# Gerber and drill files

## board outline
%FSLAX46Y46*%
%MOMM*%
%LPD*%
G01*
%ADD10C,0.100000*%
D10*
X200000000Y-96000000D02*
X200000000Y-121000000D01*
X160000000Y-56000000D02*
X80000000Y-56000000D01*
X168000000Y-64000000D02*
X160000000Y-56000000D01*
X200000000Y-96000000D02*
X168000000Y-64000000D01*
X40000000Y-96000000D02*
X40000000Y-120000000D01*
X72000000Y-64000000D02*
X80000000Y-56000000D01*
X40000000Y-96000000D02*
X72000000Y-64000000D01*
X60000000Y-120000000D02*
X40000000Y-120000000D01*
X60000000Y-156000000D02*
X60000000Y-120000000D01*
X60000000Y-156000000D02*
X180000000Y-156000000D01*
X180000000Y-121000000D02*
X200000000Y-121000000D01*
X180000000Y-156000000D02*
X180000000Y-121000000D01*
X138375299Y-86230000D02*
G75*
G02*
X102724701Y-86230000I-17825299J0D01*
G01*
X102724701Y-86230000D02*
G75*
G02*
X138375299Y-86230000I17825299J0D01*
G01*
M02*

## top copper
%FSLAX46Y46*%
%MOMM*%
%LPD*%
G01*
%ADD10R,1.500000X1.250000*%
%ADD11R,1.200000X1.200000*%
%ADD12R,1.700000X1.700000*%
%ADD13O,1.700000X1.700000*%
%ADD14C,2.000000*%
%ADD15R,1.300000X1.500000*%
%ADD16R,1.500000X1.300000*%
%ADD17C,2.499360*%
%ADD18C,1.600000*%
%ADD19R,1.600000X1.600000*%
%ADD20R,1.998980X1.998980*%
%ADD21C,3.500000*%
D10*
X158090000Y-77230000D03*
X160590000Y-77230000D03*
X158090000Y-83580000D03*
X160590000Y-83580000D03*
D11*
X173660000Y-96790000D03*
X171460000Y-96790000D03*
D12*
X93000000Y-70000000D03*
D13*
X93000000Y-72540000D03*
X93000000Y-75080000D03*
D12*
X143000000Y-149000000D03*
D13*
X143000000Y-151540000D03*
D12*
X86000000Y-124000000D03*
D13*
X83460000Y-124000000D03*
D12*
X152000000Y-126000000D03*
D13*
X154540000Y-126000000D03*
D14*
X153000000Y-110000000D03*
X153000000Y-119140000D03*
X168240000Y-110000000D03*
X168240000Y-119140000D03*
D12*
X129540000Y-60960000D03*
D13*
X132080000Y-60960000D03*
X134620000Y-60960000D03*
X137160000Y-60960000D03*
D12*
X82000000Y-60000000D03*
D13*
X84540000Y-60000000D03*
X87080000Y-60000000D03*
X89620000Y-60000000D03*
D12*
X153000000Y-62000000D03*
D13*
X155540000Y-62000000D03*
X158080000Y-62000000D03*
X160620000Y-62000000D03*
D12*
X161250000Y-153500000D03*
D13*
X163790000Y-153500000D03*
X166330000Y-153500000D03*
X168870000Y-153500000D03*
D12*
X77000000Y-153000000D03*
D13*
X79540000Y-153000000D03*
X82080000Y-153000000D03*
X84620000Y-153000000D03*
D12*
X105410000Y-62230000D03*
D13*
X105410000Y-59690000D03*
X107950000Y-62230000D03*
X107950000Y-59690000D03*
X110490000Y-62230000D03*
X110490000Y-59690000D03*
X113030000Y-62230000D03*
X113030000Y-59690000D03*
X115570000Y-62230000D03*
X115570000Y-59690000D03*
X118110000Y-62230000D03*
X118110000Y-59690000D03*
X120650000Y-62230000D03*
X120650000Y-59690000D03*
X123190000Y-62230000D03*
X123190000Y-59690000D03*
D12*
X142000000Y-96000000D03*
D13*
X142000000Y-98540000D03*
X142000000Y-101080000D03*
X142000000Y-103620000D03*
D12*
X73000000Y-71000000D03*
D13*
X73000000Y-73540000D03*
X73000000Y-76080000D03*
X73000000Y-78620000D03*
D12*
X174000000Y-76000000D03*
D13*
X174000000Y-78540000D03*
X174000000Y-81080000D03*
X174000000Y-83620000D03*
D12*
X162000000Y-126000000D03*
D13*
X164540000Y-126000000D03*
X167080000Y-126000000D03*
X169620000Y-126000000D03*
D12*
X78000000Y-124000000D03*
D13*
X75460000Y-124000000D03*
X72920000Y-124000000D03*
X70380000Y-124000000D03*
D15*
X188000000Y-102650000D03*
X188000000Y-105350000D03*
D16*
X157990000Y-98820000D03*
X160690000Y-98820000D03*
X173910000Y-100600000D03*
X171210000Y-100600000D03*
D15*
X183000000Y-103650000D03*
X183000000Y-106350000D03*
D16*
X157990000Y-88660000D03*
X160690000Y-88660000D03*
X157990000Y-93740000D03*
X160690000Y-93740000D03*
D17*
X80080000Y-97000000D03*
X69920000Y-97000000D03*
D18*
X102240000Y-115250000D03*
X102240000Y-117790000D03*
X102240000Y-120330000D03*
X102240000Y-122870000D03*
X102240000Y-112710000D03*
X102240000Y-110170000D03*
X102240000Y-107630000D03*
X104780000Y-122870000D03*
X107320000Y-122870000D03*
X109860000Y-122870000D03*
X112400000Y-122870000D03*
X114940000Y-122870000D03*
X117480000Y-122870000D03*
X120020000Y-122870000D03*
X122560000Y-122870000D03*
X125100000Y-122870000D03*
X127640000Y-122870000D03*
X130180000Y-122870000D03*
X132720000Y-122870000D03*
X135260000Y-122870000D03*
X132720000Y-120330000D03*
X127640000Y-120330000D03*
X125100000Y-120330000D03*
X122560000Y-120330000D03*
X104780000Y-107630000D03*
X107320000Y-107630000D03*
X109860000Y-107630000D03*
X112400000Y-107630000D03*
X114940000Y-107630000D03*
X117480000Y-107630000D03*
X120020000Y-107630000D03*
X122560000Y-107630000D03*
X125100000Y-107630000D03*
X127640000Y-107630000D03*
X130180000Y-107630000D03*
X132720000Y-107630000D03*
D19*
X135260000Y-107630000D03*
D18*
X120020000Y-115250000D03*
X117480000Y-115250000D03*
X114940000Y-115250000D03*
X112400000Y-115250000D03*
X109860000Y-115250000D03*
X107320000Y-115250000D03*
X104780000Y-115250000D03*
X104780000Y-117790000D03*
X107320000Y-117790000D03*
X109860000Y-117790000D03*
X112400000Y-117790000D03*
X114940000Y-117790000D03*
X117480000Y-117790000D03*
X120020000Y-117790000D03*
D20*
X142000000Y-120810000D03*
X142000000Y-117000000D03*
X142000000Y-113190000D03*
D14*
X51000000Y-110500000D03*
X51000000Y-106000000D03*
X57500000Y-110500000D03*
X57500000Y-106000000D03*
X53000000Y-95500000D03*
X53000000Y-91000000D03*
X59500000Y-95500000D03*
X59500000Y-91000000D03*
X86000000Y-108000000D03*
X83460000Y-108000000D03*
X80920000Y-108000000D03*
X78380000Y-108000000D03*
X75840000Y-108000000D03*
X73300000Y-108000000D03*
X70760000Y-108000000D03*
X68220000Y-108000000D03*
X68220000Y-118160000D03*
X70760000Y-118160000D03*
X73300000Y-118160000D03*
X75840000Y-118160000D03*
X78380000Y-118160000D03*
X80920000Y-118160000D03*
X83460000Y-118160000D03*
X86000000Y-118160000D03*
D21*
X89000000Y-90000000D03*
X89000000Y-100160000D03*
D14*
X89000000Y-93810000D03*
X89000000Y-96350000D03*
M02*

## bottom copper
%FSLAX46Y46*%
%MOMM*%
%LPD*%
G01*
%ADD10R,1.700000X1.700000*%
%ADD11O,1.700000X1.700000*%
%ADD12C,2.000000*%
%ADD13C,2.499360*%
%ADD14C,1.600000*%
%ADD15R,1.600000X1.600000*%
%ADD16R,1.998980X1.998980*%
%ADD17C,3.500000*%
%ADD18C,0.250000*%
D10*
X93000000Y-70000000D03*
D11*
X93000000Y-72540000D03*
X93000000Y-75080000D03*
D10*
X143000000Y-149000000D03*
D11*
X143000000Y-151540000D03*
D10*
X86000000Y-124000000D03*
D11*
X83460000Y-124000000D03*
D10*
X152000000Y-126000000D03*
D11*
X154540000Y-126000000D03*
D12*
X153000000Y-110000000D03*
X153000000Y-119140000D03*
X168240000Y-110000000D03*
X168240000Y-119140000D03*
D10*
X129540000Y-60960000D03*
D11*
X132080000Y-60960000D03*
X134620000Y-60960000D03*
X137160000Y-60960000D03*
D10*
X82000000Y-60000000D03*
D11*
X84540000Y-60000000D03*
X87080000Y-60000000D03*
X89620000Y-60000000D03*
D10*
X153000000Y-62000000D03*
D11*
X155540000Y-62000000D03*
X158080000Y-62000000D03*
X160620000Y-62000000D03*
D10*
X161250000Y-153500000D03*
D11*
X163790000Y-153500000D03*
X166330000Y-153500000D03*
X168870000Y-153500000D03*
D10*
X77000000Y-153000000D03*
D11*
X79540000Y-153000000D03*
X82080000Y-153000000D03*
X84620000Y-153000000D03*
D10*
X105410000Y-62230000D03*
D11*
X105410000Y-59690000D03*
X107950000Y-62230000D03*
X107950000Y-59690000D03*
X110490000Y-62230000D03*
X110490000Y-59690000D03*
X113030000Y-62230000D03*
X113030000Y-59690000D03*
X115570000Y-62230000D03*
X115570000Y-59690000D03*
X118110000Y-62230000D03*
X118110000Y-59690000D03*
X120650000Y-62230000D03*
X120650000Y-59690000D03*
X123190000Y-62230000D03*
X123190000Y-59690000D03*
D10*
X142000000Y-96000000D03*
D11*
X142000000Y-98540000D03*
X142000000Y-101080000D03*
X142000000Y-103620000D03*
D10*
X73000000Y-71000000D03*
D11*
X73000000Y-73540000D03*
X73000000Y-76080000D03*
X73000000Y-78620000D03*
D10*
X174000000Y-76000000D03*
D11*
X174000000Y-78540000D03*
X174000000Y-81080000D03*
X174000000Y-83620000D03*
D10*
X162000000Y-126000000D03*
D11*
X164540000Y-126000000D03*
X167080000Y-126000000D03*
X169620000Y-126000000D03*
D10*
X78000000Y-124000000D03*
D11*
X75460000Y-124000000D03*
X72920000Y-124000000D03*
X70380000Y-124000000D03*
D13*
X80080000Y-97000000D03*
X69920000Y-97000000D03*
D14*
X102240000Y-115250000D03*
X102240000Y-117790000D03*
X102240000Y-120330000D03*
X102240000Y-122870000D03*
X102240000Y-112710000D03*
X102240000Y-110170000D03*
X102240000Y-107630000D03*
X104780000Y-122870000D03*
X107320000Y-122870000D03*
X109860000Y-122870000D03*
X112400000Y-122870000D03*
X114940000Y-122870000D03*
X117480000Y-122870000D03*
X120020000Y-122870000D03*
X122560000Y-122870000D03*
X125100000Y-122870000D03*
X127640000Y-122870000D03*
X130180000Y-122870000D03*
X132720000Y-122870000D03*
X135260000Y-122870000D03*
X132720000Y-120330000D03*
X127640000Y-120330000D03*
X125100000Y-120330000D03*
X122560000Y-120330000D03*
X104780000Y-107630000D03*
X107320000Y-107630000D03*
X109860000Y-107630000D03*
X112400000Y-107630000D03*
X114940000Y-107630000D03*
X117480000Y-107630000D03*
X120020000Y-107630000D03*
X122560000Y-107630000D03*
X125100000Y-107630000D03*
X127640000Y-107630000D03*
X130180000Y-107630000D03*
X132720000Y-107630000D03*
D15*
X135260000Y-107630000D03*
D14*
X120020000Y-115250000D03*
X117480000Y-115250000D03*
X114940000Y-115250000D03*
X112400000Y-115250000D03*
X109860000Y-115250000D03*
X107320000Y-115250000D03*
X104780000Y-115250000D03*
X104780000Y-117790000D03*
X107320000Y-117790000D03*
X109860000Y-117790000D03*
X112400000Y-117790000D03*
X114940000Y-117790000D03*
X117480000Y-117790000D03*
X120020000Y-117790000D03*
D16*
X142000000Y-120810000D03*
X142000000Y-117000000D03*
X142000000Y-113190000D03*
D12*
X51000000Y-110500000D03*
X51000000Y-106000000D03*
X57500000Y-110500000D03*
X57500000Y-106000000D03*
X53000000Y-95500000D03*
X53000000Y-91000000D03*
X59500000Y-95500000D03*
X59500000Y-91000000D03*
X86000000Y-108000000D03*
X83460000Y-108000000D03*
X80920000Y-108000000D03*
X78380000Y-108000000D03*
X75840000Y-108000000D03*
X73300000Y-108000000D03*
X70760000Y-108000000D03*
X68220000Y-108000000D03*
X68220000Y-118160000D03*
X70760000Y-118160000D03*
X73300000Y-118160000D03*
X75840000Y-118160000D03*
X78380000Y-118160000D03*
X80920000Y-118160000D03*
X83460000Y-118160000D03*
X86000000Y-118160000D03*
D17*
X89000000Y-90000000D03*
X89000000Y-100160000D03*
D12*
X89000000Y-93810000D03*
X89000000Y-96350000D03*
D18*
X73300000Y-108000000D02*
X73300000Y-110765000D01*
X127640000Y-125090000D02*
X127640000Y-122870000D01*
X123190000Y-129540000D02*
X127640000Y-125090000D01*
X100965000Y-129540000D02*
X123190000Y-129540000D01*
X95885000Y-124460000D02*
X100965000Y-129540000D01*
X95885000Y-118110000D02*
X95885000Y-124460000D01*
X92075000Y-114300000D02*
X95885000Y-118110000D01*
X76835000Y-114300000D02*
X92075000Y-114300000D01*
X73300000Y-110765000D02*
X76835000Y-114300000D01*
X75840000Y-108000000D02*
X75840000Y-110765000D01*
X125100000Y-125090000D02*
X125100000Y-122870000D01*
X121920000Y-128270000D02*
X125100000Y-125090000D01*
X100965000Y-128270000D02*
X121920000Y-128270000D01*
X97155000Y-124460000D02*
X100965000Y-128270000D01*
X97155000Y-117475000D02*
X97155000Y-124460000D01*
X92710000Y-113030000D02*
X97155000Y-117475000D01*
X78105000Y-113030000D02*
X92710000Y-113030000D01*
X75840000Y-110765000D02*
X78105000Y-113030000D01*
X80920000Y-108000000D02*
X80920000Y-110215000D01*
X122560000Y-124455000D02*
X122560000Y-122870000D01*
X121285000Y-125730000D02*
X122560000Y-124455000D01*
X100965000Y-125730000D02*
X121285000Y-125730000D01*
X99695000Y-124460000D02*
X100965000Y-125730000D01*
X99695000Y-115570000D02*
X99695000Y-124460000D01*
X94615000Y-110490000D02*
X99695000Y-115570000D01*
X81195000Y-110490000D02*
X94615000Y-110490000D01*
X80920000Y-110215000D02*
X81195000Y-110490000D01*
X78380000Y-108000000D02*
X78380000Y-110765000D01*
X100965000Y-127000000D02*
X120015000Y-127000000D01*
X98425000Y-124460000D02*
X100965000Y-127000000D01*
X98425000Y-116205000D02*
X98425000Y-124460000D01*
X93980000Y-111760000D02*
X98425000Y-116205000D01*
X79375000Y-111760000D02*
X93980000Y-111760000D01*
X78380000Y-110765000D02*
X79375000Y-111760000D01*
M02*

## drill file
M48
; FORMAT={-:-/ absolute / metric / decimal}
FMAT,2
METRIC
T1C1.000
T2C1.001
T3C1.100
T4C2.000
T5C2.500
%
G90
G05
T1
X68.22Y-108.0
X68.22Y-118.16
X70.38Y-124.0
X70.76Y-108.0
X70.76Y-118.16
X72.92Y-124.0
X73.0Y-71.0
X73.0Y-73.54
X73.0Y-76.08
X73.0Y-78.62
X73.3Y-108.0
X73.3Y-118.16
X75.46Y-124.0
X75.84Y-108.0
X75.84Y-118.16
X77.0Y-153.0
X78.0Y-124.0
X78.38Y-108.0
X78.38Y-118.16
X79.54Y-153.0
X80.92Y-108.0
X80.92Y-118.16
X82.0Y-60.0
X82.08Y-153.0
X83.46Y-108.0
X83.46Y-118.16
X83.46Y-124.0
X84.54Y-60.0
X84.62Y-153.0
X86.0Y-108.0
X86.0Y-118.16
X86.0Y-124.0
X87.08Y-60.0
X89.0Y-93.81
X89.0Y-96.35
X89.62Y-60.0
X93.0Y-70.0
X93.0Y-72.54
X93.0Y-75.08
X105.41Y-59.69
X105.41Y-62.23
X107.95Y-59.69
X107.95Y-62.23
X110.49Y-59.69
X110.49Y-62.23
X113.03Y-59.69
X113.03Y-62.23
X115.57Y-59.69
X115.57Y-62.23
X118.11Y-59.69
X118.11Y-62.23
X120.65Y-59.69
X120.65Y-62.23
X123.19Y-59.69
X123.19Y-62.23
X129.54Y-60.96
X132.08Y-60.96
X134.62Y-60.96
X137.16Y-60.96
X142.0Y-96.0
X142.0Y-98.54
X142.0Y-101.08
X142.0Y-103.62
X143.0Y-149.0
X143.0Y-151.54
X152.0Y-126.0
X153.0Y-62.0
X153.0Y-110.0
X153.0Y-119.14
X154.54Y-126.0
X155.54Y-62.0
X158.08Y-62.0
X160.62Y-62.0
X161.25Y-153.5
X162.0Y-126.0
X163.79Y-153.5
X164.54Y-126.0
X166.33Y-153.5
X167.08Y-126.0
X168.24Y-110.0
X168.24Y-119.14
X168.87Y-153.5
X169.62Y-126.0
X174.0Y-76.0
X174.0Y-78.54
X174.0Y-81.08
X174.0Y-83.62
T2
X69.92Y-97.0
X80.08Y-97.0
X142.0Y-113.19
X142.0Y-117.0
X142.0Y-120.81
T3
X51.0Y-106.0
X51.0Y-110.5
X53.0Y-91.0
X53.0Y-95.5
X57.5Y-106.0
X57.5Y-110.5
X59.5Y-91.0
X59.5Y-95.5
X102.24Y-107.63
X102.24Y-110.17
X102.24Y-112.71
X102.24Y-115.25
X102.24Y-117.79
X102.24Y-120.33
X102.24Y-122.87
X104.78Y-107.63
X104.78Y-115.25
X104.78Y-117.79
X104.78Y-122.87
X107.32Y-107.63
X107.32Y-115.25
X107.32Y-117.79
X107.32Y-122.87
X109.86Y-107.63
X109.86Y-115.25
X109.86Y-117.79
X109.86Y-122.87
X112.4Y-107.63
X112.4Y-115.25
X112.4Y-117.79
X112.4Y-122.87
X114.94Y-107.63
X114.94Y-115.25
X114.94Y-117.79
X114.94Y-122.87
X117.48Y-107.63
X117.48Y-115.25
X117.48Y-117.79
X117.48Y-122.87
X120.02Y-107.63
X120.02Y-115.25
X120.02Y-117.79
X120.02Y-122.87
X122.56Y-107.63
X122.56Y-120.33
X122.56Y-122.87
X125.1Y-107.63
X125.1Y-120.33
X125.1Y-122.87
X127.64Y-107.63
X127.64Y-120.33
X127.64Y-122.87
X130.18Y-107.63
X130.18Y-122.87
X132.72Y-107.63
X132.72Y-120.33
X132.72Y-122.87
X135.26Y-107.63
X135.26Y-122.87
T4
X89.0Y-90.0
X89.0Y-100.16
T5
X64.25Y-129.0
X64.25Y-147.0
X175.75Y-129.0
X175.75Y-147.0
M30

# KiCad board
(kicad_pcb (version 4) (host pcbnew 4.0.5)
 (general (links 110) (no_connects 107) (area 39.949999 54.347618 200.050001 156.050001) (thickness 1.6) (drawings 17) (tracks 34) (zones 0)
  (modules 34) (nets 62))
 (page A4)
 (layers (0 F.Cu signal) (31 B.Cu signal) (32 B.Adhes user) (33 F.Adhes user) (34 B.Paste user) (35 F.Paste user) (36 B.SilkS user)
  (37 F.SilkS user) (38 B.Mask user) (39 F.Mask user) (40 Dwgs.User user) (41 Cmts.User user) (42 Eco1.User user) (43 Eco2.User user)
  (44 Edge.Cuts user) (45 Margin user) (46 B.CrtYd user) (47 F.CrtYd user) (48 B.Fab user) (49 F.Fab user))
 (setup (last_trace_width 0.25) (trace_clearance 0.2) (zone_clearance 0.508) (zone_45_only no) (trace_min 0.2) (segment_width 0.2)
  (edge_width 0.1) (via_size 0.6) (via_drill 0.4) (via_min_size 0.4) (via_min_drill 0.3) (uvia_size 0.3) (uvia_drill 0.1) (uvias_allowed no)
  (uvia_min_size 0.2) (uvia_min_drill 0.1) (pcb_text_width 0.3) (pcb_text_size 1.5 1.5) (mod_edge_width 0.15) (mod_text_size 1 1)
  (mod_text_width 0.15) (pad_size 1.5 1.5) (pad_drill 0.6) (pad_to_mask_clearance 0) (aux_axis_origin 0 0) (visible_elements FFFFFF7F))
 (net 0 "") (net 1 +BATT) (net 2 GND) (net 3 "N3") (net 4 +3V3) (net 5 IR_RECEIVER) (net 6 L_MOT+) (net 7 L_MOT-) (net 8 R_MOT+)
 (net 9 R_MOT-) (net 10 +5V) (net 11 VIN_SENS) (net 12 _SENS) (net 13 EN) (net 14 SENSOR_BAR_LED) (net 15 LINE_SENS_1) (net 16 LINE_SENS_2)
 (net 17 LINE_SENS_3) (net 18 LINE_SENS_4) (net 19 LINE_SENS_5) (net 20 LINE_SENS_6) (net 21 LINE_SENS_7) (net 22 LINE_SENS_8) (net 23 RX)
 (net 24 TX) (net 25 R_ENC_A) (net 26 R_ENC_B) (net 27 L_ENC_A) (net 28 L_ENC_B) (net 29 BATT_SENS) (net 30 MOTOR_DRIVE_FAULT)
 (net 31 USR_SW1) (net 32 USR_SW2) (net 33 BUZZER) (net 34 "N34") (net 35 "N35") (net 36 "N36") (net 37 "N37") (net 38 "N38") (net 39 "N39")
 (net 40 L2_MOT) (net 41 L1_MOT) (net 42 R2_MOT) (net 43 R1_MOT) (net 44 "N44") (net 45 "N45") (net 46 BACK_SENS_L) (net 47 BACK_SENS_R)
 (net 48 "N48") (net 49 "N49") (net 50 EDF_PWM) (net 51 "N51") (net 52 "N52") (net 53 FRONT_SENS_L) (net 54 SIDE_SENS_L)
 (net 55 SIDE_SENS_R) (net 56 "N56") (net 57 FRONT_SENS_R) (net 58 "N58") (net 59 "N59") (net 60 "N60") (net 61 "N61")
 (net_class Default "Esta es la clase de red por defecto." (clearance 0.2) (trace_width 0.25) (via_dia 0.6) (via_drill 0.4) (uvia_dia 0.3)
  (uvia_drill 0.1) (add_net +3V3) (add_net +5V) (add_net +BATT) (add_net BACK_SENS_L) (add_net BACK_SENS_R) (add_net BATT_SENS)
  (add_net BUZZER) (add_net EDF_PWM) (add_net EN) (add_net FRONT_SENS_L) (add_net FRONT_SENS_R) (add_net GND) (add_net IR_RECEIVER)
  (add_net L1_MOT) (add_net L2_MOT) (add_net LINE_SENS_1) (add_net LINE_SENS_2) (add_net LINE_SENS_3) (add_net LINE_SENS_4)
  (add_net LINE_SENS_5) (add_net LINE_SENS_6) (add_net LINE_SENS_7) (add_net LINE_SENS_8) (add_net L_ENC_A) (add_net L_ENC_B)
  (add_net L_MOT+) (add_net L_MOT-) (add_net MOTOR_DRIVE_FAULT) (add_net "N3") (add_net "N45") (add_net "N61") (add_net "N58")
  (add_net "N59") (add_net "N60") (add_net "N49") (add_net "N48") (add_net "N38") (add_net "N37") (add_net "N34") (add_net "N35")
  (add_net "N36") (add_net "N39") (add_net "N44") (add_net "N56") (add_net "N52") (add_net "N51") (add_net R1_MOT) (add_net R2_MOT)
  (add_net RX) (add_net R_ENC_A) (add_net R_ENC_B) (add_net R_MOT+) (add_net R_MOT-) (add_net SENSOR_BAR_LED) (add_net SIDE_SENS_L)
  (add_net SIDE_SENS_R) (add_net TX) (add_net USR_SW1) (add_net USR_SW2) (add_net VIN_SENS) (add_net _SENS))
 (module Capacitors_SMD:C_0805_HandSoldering (layer F.Cu) (at 159.34 77.23)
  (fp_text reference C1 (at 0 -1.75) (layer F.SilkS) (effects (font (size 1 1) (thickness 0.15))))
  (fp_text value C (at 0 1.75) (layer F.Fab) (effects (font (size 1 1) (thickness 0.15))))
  (pad 1 smd rect (at -1.25 0) (size 1.5 1.25) (layers F.Cu F.Paste F.Mask) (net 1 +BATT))
  (pad 2 smd rect (at 1.25 0) (size 1.5 1.25) (layers F.Cu F.Paste F.Mask) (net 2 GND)))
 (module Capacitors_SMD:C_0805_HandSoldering (layer F.Cu) (at 159.34 83.58)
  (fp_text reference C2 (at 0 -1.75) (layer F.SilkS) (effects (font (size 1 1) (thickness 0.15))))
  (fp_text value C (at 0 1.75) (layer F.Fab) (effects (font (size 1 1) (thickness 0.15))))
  (pad 1 smd rect (at -1.25 0) (size 1.5 1.25) (layers F.Cu F.Paste F.Mask) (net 1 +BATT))
  (pad 2 smd rect (at 1.25 0) (size 1.5 1.25) (layers F.Cu F.Paste F.Mask) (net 2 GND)))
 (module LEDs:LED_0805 (layer F.Cu) (at 172.56 96.79)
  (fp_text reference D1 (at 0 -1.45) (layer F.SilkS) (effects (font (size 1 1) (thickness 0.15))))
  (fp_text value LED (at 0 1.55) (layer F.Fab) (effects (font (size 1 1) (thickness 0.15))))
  (pad 2 smd rect (at 1.1 0 180) (size 1.2 1.2) (layers F.Cu F.Paste F.Mask) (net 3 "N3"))
  (pad 1 smd rect (at -1.1 0 180) (size 1.2 1.2) (layers F.Cu F.Paste F.Mask) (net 1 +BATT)))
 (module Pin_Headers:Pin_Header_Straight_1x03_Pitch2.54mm (layer F.Cu) (at 93 70)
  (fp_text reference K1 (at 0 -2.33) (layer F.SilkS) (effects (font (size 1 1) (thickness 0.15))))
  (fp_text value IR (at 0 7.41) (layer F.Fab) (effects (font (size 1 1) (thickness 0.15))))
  (pad 1 thru_hole rect (at 0 0) (size 1.7 1.7) (drill 1) (layers *.Cu *.Mask) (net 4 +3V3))
  (pad 2 thru_hole oval (at 0 2.54) (size 1.7 1.7) (drill 1) (layers *.Cu *.Mask) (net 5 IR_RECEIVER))
  (pad 3 thru_hole oval (at 0 5.08) (size 1.7 1.7) (drill 1) (layers *.Cu *.Mask) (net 2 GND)))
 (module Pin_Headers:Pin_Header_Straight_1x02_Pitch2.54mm (layer F.Cu) (at 143 149)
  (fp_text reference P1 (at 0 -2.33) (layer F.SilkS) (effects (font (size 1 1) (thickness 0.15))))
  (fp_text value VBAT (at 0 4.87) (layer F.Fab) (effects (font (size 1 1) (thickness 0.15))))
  (pad 1 thru_hole rect (at 0 0) (size 1.7 1.7) (drill 1) (layers *.Cu *.Mask) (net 1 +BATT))
  (pad 2 thru_hole oval (at 0 2.54) (size 1.7 1.7) (drill 1) (layers *.Cu *.Mask) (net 2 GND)))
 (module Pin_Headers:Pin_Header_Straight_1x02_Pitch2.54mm (layer F.Cu) (at 86 124 270)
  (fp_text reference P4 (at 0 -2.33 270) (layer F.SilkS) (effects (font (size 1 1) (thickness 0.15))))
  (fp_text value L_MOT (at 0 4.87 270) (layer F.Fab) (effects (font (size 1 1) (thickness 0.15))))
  (pad 1 thru_hole rect (at 0 0 270) (size 1.7 1.7) (drill 1) (layers *.Cu *.Mask) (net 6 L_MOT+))
  (pad 2 thru_hole oval (at 0 2.54 270) (size 1.7 1.7) (drill 1) (layers *.Cu *.Mask) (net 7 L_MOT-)))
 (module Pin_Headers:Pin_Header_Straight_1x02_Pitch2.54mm (layer F.Cu) (at 152 126 90)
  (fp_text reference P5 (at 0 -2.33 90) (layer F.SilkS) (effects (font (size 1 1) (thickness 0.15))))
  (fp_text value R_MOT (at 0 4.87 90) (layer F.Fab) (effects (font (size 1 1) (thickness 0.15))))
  (pad 1 thru_hole rect (at 0 0 90) (size 1.7 1.7) (drill 1) (layers *.Cu *.Mask) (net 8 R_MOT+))
  (pad 2 thru_hole oval (at 0 2.54 90) (size 1.7 1.7) (drill 1) (layers *.Cu *.Mask) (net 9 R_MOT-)))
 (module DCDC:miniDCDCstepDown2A (layer F.Cu) (at 153 110)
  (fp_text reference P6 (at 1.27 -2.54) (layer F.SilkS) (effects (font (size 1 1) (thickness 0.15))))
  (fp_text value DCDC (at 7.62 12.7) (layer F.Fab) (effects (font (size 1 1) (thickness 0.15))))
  (pad 2 thru_hole circle (at 0 0) (size 2 2) (drill 1) (layers *.Cu *.Mask) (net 2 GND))
  (pad 1 thru_hole circle (at 0 9.14) (size 2 2) (drill 1) (layers *.Cu *.Mask) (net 1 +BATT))
  (pad 4 thru_hole circle (at 15.24 0) (size 2 2) (drill 1) (layers *.Cu *.Mask) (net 2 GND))
  (pad 3 thru_hole circle (at 15.24 9.14) (size 2 2) (drill 1) (layers *.Cu *.Mask) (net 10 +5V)))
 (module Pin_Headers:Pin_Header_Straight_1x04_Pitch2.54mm (layer F.Cu) (at 129.54 60.96 90)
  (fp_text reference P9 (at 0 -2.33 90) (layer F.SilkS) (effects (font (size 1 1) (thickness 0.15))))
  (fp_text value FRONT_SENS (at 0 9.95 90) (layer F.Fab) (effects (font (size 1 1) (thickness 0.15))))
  (pad 1 thru_hole rect (at 0 0 90) (size 1.7 1.7) (drill 1) (layers *.Cu *.Mask) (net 2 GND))
  (pad 2 thru_hole oval (at 0 2.54 90) (size 1.7 1.7) (drill 1) (layers *.Cu *.Mask) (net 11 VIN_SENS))
  (pad 3 thru_hole oval (at 0 5.08 90) (size 1.7 1.7) (drill 1) (layers *.Cu *.Mask) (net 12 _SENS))
  (pad 4 thru_hole oval (at 0 7.62 90) (size 1.7 1.7) (drill 1) (layers *.Cu *.Mask) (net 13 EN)))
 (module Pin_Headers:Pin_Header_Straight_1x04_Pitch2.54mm (layer F.Cu) (at 82 60 90)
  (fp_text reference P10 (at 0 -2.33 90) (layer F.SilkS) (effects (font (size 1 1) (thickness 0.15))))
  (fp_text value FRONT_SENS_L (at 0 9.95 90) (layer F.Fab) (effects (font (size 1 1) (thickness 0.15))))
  (pad 1 thru_hole rect (at 0 0 90) (size 1.7 1.7) (drill 1) (layers *.Cu *.Mask) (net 2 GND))
  (pad 2 thru_hole oval (at 0 2.54 90) (size 1.7 1.7) (drill 1) (layers *.Cu *.Mask) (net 11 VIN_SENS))
  (pad 3 thru_hole oval (at 0 5.08 90) (size 1.7 1.7) (drill 1) (layers *.Cu *.Mask) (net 12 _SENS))
  (pad 4 thru_hole oval (at 0 7.62 90) (size 1.7 1.7) (drill 1) (layers *.Cu *.Mask) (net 13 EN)))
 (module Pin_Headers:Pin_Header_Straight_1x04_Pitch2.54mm (layer F.Cu) (at 153 62 90)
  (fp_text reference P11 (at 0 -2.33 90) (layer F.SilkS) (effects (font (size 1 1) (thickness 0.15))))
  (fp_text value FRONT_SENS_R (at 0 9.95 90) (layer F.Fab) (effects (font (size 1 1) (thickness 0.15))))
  (pad 1 thru_hole rect (at 0 0 90) (size 1.7 1.7) (drill 1) (layers *.Cu *.Mask) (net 2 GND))
  (pad 2 thru_hole oval (at 0 2.54 90) (size 1.7 1.7) (drill 1) (layers *.Cu *.Mask) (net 11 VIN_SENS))
  (pad 3 thru_hole oval (at 0 5.08 90) (size 1.7 1.7) (drill 1) (layers *.Cu *.Mask) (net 12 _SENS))
  (pad 4 thru_hole oval (at 0 7.62 90) (size 1.7 1.7) (drill 1) (layers *.Cu *.Mask) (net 13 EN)))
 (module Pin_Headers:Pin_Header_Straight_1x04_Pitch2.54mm (layer F.Cu) (at 161.25 153.5 90)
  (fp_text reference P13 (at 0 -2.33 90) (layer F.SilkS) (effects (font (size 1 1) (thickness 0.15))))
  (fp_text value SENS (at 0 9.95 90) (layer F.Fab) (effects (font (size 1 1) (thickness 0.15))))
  (pad 1 thru_hole rect (at 0 0 90) (size 1.7 1.7) (drill 1) (layers *.Cu *.Mask) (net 2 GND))
  (pad 2 thru_hole oval (at 0 2.54 90) (size 1.7 1.7) (drill 1) (layers *.Cu *.Mask) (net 11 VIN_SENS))
  (pad 3 thru_hole oval (at 0 5.08 90) (size 1.7 1.7) (drill 1) (layers *.Cu *.Mask) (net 12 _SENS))
  (pad 4 thru_hole oval (at 0 7.62 90) (size 1.7 1.7) (drill 1) (layers *.Cu *.Mask) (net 13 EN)))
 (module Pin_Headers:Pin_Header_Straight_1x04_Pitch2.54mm (layer F.Cu) (at 77 153 90)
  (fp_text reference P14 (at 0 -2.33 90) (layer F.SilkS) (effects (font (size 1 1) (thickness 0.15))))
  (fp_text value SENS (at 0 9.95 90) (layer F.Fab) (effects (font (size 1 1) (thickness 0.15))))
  (pad 1 thru_hole rect (at 0 0 90) (size 1.7 1.7) (drill 1) (layers *.Cu *.Mask) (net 2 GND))
  (pad 2 thru_hole oval (at 0 2.54 90) (size 1.7 1.7) (drill 1) (layers *.Cu *.Mask) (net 11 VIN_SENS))
  (pad 3 thru_hole oval (at 0 5.08 90) (size 1.7 1.7) (drill 1) (layers *.Cu *.Mask) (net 12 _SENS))
  (pad 4 thru_hole oval (at 0 7.62 90) (size 1.7 1.7) (drill 1) (layers *.Cu *.Mask) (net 13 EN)))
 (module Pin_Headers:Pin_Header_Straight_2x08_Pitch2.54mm (layer F.Cu) (at 105.41 62.23 90)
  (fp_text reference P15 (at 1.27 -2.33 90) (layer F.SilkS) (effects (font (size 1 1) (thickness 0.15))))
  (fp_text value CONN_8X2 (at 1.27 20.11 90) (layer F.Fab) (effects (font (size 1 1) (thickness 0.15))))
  (pad 1 thru_hole rect (at 0 0 90) (size 1.7 1.7) (drill 1) (layers *.Cu *.Mask) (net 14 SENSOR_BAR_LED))
  (pad 2 thru_hole oval (at 2.54 0 90) (size 1.7 1.7) (drill 1) (layers *.Cu *.Mask) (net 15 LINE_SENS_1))
  (pad 3 thru_hole oval (at 0 2.54 90) (size 1.7 1.7) (drill 1) (layers *.Cu *.Mask) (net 4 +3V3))
  (pad 4 thru_hole oval (at 2.54 2.54 90) (size 1.7 1.7) (drill 1) (layers *.Cu *.Mask) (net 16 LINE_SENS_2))
  (pad 5 thru_hole oval (at 0 5.08 90) (size 1.7 1.7) (drill 1) (layers *.Cu *.Mask) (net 2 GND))
  (pad 6 thru_hole oval (at 2.54 5.08 90) (size 1.7 1.7) (drill 1) (layers *.Cu *.Mask) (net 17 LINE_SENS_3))
  (pad 7 thru_hole oval (at 0 7.62 90) (size 1.7 1.7) (drill 1) (layers *.Cu *.Mask) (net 2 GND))
  (pad 8 thru_hole oval (at 2.54 7.62 90) (size 1.7 1.7) (drill 1) (layers *.Cu *.Mask) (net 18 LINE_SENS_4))
  (pad 9 thru_hole oval (at 0 10.16 90) (size 1.7 1.7) (drill 1) (layers *.Cu *.Mask) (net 2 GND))
  (pad 10 thru_hole oval (at 2.54 10.16 90) (size 1.7 1.7) (drill 1) (layers *.Cu *.Mask) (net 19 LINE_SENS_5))
  (pad 11 thru_hole oval (at 0 12.7 90) (size 1.7 1.7) (drill 1) (layers *.Cu *.Mask) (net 2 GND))
  (pad 12 thru_hole oval (at 2.54 12.7 90) (size 1.7 1.7) (drill 1) (layers *.Cu *.Mask) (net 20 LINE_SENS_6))
  (pad 13 thru_hole oval (at 0 15.24 90) (size 1.7 1.7) (drill 1) (layers *.Cu *.Mask) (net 2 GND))
  (pad 14 thru_hole oval (at 2.54 15.24 90) (size 1.7 1.7) (drill 1) (layers *.Cu *.Mask) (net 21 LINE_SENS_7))
  (pad 15 thru_hole oval (at 0 17.78 90) (size 1.7 1.7) (drill 1) (layers *.Cu *.Mask) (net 2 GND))
  (pad 16 thru_hole oval (at 2.54 17.78 90) (size 1.7 1.7) (drill 1) (layers *.Cu *.Mask) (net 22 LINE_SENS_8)))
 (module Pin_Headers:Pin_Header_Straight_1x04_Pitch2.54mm (layer F.Cu) (at 142 96)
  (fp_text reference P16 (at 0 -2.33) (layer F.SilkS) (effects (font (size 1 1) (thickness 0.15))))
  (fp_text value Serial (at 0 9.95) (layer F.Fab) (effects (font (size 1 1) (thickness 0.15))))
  (pad 1 thru_hole rect (at 0 0) (size 1.7 1.7) (drill 1) (layers *.Cu *.Mask) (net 10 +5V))
  (pad 2 thru_hole oval (at 0 2.54) (size 1.7 1.7) (drill 1) (layers *.Cu *.Mask) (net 2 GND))
  (pad 3 thru_hole oval (at 0 5.08) (size 1.7 1.7) (drill 1) (layers *.Cu *.Mask) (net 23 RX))
  (pad 4 thru_hole oval (at 0 7.62) (size 1.7 1.7) (drill 1) (layers *.Cu *.Mask) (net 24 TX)))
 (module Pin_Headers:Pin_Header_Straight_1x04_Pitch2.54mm (layer F.Cu) (at 73 71)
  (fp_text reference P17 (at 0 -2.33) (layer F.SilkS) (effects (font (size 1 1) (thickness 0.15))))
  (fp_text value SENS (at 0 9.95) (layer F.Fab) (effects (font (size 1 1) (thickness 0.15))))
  (pad 1 thru_hole rect (at 0 0) (size 1.7 1.7) (drill 1) (layers *.Cu *.Mask) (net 2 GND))
  (pad 2 thru_hole oval (at 0 2.54) (size 1.7 1.7) (drill 1) (layers *.Cu *.Mask) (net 11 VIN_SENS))
  (pad 3 thru_hole oval (at 0 5.08) (size 1.7 1.7) (drill 1) (layers *.Cu *.Mask) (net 12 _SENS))
  (pad 4 thru_hole oval (at 0 7.62) (size 1.7 1.7) (drill 1) (layers *.Cu *.Mask) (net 13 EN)))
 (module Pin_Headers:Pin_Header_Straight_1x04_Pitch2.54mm (layer F.Cu) (at 174 76)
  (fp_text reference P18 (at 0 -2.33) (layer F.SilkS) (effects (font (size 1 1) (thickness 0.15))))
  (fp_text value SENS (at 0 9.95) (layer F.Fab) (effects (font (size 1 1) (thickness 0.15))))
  (pad 1 thru_hole rect (at 0 0) (size 1.7 1.7) (drill 1) (layers *.Cu *.Mask) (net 2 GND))
  (pad 2 thru_hole oval (at 0 2.54) (size 1.7 1.7) (drill 1) (layers *.Cu *.Mask) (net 11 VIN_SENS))
  (pad 3 thru_hole oval (at 0 5.08) (size 1.7 1.7) (drill 1) (layers *.Cu *.Mask) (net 12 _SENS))
  (pad 4 thru_hole oval (at 0 7.62) (size 1.7 1.7) (drill 1) (layers *.Cu *.Mask) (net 13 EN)))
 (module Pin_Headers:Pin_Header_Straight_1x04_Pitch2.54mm (layer F.Cu) (at 162 126 90)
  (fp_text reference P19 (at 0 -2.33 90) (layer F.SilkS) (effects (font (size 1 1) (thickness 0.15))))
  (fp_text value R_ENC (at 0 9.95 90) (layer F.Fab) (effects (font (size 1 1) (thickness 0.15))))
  (pad 1 thru_hole rect (at 0 0 90) (size 1.7 1.7) (drill 1) (layers *.Cu *.Mask) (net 4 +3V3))
  (pad 2 thru_hole oval (at 0 2.54 90) (size 1.7 1.7) (drill 1) (layers *.Cu *.Mask) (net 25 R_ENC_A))
  (pad 3 thru_hole oval (at 0 5.08 90) (size 1.7 1.7) (drill 1) (layers *.Cu *.Mask) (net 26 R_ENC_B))
  (pad 4 thru_hole oval (at 0 7.62 90) (size 1.7 1.7) (drill 1) (layers *.Cu *.Mask) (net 2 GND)))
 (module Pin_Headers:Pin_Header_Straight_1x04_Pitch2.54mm (layer F.Cu) (at 78 124 270)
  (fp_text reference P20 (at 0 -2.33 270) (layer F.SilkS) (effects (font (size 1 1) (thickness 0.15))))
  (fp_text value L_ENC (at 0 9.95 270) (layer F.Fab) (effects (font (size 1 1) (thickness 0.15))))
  (pad 1 thru_hole rect (at 0 0 270) (size 1.7 1.7) (drill 1) (layers *.Cu *.Mask) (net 4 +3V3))
  (pad 2 thru_hole oval (at 0 2.54 270) (size 1.7 1.7) (drill 1) (layers *.Cu *.Mask) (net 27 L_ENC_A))
  (pad 3 thru_hole oval (at 0 5.08 270) (size 1.7 1.7) (drill 1) (layers *.Cu *.Mask) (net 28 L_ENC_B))
  (pad 4 thru_hole oval (at 0 7.62 270) (size 1.7 1.7) (drill 1) (layers *.Cu *.Mask) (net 2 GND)))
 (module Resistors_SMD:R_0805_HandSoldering (layer F.Cu) (at 188 104 270)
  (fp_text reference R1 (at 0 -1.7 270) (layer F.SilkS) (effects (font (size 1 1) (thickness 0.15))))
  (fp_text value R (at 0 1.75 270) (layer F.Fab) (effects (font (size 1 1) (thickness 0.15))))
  (pad 1 smd rect (at -1.35 0 270) (size 1.5 1.3) (layers F.Cu F.Paste F.Mask) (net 1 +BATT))
  (pad 2 smd rect (at 1.35 0 270) (size 1.5 1.3) (layers F.Cu F.Paste F.Mask) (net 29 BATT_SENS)))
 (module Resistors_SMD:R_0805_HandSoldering (layer F.Cu) (at 159.34 98.82)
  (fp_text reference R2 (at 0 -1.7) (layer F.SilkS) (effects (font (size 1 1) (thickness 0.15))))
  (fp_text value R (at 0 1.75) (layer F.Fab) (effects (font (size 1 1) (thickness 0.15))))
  (pad 1 smd rect (at -1.35 0) (size 1.5 1.3) (layers F.Cu F.Paste F.Mask) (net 4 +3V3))
  (pad 2 smd rect (at 1.35 0) (size 1.5 1.3) (layers F.Cu F.Paste F.Mask) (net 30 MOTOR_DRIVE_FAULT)))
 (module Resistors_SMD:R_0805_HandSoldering (layer F.Cu) (at 172.56 100.6 180)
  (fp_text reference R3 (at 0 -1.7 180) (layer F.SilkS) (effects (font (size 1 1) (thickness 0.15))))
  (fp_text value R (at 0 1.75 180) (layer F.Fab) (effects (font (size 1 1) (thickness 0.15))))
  (pad 1 smd rect (at -1.35 0 180) (size 1.5 1.3) (layers F.Cu F.Paste F.Mask) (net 3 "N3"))
  (pad 2 smd rect (at 1.35 0 180) (size 1.5 1.3) (layers F.Cu F.Paste F.Mask) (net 2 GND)))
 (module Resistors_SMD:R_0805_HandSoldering (layer F.Cu) (at 183 105 270)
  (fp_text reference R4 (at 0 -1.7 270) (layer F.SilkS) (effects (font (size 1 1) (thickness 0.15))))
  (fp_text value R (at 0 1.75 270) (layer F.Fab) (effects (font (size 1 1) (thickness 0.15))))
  (pad 1 smd rect (at -1.35 0 270) (size 1.5 1.3) (layers F.Cu F.Paste F.Mask) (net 29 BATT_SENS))
  (pad 2 smd rect (at 1.35 0 270) (size 1.5 1.3) (layers F.Cu F.Paste F.Mask) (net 2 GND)))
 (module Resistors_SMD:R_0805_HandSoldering (layer F.Cu) (at 159.34 88.66)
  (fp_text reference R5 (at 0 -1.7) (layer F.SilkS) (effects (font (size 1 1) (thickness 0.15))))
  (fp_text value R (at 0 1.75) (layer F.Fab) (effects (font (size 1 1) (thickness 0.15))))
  (pad 1 smd rect (at -1.35 0) (size 1.5 1.3) (layers F.Cu F.Paste F.Mask) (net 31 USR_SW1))
  (pad 2 smd rect (at 1.35 0) (size 1.5 1.3) (layers F.Cu F.Paste F.Mask) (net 2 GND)))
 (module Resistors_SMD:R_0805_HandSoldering (layer F.Cu) (at 159.34 93.74)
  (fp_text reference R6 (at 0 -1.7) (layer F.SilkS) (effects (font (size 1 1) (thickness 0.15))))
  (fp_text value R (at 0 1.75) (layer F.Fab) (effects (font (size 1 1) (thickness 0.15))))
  (pad 1 smd rect (at -1.35 0) (size 1.5 1.3) (layers F.Cu F.Paste F.Mask) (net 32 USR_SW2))
  (pad 2 smd rect (at 1.35 0) (size 1.5 1.3) (layers F.Cu F.Paste F.Mask) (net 2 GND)))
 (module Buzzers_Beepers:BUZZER (layer F.Cu) (at 75 97)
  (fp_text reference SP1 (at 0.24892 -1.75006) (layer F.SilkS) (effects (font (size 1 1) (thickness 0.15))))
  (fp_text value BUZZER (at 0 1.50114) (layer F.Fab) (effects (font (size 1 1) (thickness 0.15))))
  (pad 2 thru_hole circle (at 5.08 0) (size 2.49936 2.49936) (drill 1.00076) (layers *.Cu *.Mask) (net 2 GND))
  (pad 1 thru_hole circle (at -5.08 0) (size 2.49936 2.49936) (drill 1.00076) (layers *.Cu *.Mask) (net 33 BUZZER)))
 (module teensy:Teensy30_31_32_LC (layer F.Cu) (at 118.75 115.25 180)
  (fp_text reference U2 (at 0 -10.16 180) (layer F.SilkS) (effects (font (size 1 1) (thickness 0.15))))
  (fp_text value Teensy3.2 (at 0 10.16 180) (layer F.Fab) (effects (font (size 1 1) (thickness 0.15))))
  (pad 17 thru_hole circle (at 16.51 0 180) (size 1.6 1.6) (drill 1.1) (layers *.Cu *.Mask F.SilkS) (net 2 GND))
  (pad 18 thru_hole circle (at 16.51 -2.54 180) (size 1.6 1.6) (drill 1.1) (layers *.Cu *.Mask F.SilkS) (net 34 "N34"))
  (pad 19 thru_hole circle (at 16.51 -5.08 180) (size 1.6 1.6) (drill 1.1) (layers *.Cu *.Mask F.SilkS) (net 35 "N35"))
  (pad 20 thru_hole circle (at 16.51 -7.62 180) (size 1.6 1.6) (drill 1.1) (layers *.Cu *.Mask F.SilkS) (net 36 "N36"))
  (pad 16 thru_hole circle (at 16.51 2.54 180) (size 1.6 1.6) (drill 1.1) (layers *.Cu *.Mask F.SilkS) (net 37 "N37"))
  (pad 15 thru_hole circle (at 16.51 5.08 180) (size 1.6 1.6) (drill 1.1) (layers *.Cu *.Mask F.SilkS) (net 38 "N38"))
  (pad 14 thru_hole circle (at 16.51 7.62 180) (size 1.6 1.6) (drill 1.1) (layers *.Cu *.Mask F.SilkS) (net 30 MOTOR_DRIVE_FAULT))
  (pad 21 thru_hole circle (at 13.97 -7.62 180) (size 1.6 1.6) (drill 1.1) (layers *.Cu *.Mask F.SilkS) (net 29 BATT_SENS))
  (pad 22 thru_hole circle (at 11.43 -7.62 180) (size 1.6 1.6) (drill 1.1) (layers *.Cu *.Mask F.SilkS) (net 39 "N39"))
  (pad 23 thru_hole circle (at 8.89 -7.62 180) (size 1.6 1.6) (drill 1.1) (layers *.Cu *.Mask F.SilkS) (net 15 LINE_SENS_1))
  (pad 24 thru_hole circle (at 6.35 -7.62 180) (size 1.6 1.6) (drill 1.1) (layers *.Cu *.Mask F.SilkS) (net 16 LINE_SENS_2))
  (pad 25 thru_hole circle (at 3.81 -7.62 180) (size 1.6 1.6) (drill 1.1) (layers *.Cu *.Mask F.SilkS) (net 17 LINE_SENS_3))
  (pad 26 thru_hole circle (at 1.27 -7.62 180) (size 1.6 1.6) (drill 1.1) (layers *.Cu *.Mask F.SilkS) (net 18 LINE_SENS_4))
  (pad 27 thru_hole circle (at -1.27 -7.62 180) (size 1.6 1.6) (drill 1.1) (layers *.Cu *.Mask F.SilkS) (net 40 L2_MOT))
  (pad 28 thru_hole circle (at -3.81 -7.62 180) (size 1.6 1.6) (drill 1.1) (layers *.Cu *.Mask F.SilkS) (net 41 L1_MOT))
  (pad 29 thru_hole circle (at -6.35 -7.62 180) (size 1.6 1.6) (drill 1.1) (layers *.Cu *.Mask F.SilkS) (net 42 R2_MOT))
  (pad 30 thru_hole circle (at -8.89 -7.62 180) (size 1.6 1.6) (drill 1.1) (layers *.Cu *.Mask F.SilkS) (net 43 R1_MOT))
  (pad 31 thru_hole circle (at -11.43 -7.62 180) (size 1.6 1.6) (drill 1.1) (layers *.Cu *.Mask F.SilkS) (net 4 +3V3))
  (pad 32 thru_hole circle (at -13.97 -7.62 180) (size 1.6 1.6) (drill 1.1) (layers *.Cu *.Mask F.SilkS) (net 2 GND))
  (pad 33 thru_hole circle (at -16.51 -7.62 180) (size 1.6 1.6) (drill 1.1) (layers *.Cu *.Mask F.SilkS) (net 10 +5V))
  (pad 34 thru_hole circle (at -13.97 -5.08 180) (size 1.6 1.6) (drill 1.1) (layers *.Cu *.Mask F.SilkS) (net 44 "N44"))
  (pad 35 thru_hole circle (at -8.89 -5.08 180) (size 1.6 1.6) (drill 1.1) (layers *.Cu *.Mask F.SilkS) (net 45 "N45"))
  (pad 36 thru_hole circle (at -6.35 -5.08 180) (size 1.6 1.6) (drill 1.1) (layers *.Cu *.Mask F.SilkS) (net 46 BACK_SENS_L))
  (pad 37 thru_hole circle (at -3.81 -5.08 180) (size 1.6 1.6) (drill 1.1) (layers *.Cu *.Mask F.SilkS) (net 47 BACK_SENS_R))
  (pad 13 thru_hole circle (at 13.97 7.62 180) (size 1.6 1.6) (drill 1.1) (layers *.Cu *.Mask F.SilkS) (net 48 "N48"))
  (pad 12 thru_hole circle (at 11.43 7.62 180) (size 1.6 1.6) (drill 1.1) (layers *.Cu *.Mask F.SilkS) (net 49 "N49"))
  (pad 11 thru_hole circle (at 8.89 7.62 180) (size 1.6 1.6) (drill 1.1) (layers *.Cu *.Mask F.SilkS) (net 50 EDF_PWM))
  (pad 10 thru_hole circle (at 6.35 7.62 180) (size 1.6 1.6) (drill 1.1) (layers *.Cu *.Mask F.SilkS) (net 14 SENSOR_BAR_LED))
  (pad 9 thru_hole circle (at 3.81 7.62 180) (size 1.6 1.6) (drill 1.1) (layers *.Cu *.Mask F.SilkS) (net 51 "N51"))
  (pad 8 thru_hole circle (at 1.27 7.62 180) (size 1.6 1.6) (drill 1.1) (layers *.Cu *.Mask F.SilkS) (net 33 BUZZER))
  (pad 7 thru_hole circle (at -1.27 7.62 180) (size 1.6 1.6) (drill 1.1) (layers *.Cu *.Mask F.SilkS) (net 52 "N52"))
  (pad 6 thru_hole circle (at -3.81 7.62 180) (size 1.6 1.6) (drill 1.1) (layers *.Cu *.Mask F.SilkS) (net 26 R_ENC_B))
  (pad 5 thru_hole circle (at -6.35 7.62 180) (size 1.6 1.6) (drill 1.1) (layers *.Cu *.Mask F.SilkS) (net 25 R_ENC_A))
  (pad 4 thru_hole circle (at -8.89 7.62 180) (size 1.6 1.6) (drill 1.1) (layers *.Cu *.Mask F.SilkS) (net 5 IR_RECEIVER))
  (pad 3 thru_hole circle (at -11.43 7.62 180) (size 1.6 1.6) (drill 1.1) (layers *.Cu *.Mask F.SilkS) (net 24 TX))
  (pad 2 thru_hole circle (at -13.97 7.62 180) (size 1.6 1.6) (drill 1.1) (layers *.Cu *.Mask F.SilkS) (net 23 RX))
  (pad 1 thru_hole rect (at -16.51 7.62 180) (size 1.6 1.6) (drill 1.1) (layers *.Cu *.Mask F.SilkS) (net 2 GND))
  (pad 38 thru_hole circle (at -1.27 0 180) (size 1.6 1.6) (drill 1.1) (layers *.Cu *.Mask) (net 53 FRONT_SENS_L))
  (pad 39 thru_hole circle (at 1.27 0 180) (size 1.6 1.6) (drill 1.1) (layers *.Cu *.Mask) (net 2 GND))
  (pad 40 thru_hole circle (at 3.81 0 180) (size 1.6 1.6) (drill 1.1) (layers *.Cu *.Mask) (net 32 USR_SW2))
  (pad 41 thru_hole circle (at 6.35 0 180) (size 1.6 1.6) (drill 1.1) (layers *.Cu *.Mask) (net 28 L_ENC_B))
  (pad 42 thru_hole circle (at 8.89 0 180) (size 1.6 1.6) (drill 1.1) (layers *.Cu *.Mask) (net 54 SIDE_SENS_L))
  (pad 43 thru_hole circle (at 11.43 0 180) (size 1.6 1.6) (drill 1.1) (layers *.Cu *.Mask) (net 22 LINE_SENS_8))
  (pad 44 thru_hole circle (at 13.97 0 180) (size 1.6 1.6) (drill 1.1) (layers *.Cu *.Mask) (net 20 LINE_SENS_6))
  (pad 45 thru_hole circle (at 13.97 -2.54 180) (size 1.6 1.6) (drill 1.1) (layers *.Cu *.Mask) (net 19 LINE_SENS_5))
  (pad 46 thru_hole circle (at 11.43 -2.54 180) (size 1.6 1.6) (drill 1.1) (layers *.Cu *.Mask) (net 21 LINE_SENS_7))
  (pad 47 thru_hole circle (at 8.89 -2.54 180) (size 1.6 1.6) (drill 1.1) (layers *.Cu *.Mask) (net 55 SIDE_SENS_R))
  (pad 48 thru_hole circle (at 6.35 -2.54 180) (size 1.6 1.6) (drill 1.1) (layers *.Cu *.Mask) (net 27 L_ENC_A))
  (pad 49 thru_hole circle (at 3.81 -2.54 180) (size 1.6 1.6) (drill 1.1) (layers *.Cu *.Mask) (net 31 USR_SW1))
  (pad 50 thru_hole circle (at 1.27 -2.54 180) (size 1.6 1.6) (drill 1.1) (layers *.Cu *.Mask) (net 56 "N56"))
  (pad 51 thru_hole circle (at -1.27 -2.54 180) (size 1.6 1.6) (drill 1.1) (layers *.Cu *.Mask) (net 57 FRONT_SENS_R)))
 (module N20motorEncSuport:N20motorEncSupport (layer F.Cu) (at 60 138)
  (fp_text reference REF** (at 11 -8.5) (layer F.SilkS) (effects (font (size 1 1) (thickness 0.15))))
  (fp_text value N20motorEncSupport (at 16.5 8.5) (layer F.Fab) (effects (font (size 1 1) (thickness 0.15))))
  (pad "" np_thru_hole circle (at 4.25 -9) (size 2.5 2.5) (drill 2.5) (layers *.Cu *.Mask))
  (pad "" np_thru_hole circle (at 4.25 9) (size 2.5 2.5) (drill 2.5) (layers *.Cu *.Mask)))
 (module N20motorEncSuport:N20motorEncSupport (layer F.Cu) (at 180 138 180)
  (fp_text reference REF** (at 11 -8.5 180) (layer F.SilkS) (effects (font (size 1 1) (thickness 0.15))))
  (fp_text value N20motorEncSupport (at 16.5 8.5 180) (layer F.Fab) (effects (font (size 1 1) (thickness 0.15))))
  (pad "" np_thru_hole circle (at 4.25 -9 180) (size 2.5 2.5) (drill 2.5) (layers *.Cu *.Mask))
  (pad "" np_thru_hole circle (at 4.25 9 180) (size 2.5 2.5) (drill 2.5) (layers *.Cu *.Mask)))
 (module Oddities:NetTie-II (layer F.Cu) (at 142 117 90)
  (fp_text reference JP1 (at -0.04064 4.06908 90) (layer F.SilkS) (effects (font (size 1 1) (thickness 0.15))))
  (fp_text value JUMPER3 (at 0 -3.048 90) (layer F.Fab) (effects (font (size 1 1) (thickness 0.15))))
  (pad 1 thru_hole rect (at -3.81 0 90) (size 1.99898 1.99898) (drill 1.00076) (layers *.Cu *.Mask) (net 10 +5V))
  (pad 2 thru_hole rect (at 0 0 90) (size 1.99898 1.99898) (drill 1.00076) (layers *.Cu *.Mask) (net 45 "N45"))
  (pad 3 thru_hole rect (at 3.81 0 90) (size 1.99898 1.99898) (drill 1.00076) (layers *.Cu *.Mask) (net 4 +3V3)))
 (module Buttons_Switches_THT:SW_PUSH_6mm (layer F.Cu) (at 51 106)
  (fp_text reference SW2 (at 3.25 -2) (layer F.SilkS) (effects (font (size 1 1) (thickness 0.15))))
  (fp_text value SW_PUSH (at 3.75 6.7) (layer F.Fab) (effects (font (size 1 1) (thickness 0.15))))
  (pad 2 thru_hole circle (at 0 4.5 90) (size 2 2) (drill 1.1) (layers *.Cu *.Mask) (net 31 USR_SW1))
  (pad 1 thru_hole circle (at 0 0 90) (size 2 2) (drill 1.1) (layers *.Cu *.Mask) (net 4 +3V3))
  (pad 2 thru_hole circle (at 6.5 4.5 90) (size 2 2) (drill 1.1) (layers *.Cu *.Mask) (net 31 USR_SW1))
  (pad 1 thru_hole circle (at 6.5 0 90) (size 2 2) (drill 1.1) (layers *.Cu *.Mask) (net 4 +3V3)))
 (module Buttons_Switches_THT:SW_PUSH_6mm (layer F.Cu) (at 53 91)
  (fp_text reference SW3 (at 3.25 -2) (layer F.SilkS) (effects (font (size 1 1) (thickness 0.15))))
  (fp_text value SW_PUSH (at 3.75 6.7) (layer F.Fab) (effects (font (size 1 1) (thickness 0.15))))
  (pad 2 thru_hole circle (at 0 4.5 90) (size 2 2) (drill 1.1) (layers *.Cu *.Mask) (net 32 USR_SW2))
  (pad 1 thru_hole circle (at 0 0 90) (size 2 2) (drill 1.1) (layers *.Cu *.Mask) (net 4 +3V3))
  (pad 2 thru_hole circle (at 6.5 4.5 90) (size 2 2) (drill 1.1) (layers *.Cu *.Mask) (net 32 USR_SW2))
  (pad 1 thru_hole circle (at 6.5 0 90) (size 2 2) (drill 1.1) (layers *.Cu *.Mask) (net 4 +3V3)))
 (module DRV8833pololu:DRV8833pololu (layer F.Cu) (at 86 108 180)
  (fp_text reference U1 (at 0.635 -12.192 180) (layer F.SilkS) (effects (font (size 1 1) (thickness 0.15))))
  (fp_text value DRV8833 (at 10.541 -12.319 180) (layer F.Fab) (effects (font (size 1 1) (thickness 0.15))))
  (pad 1 thru_hole circle (at 0 0 180) (size 2 2) (drill 1) (layers *.Cu *.Mask) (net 2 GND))
  (pad 2 thru_hole circle (at 2.54 0 180) (size 2 2) (drill 1) (layers *.Cu *.Mask) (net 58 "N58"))
  (pad 3 thru_hole circle (at 5.08 0 180) (size 2 2) (drill 1) (layers *.Cu *.Mask) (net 41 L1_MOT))
  (pad 4 thru_hole circle (at 7.62 0 180) (size 2 2) (drill 1) (layers *.Cu *.Mask) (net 40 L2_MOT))
  (pad 5 thru_hole circle (at 10.16 0 180) (size 2 2) (drill 1) (layers *.Cu *.Mask) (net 42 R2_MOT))
  (pad 6 thru_hole circle (at 12.7 0 180) (size 2 2) (drill 1) (layers *.Cu *.Mask) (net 43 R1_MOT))
  (pad 7 thru_hole circle (at 15.24 0 180) (size 2 2) (drill 1) (layers *.Cu *.Mask) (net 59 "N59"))
  (pad 8 thru_hole circle (at 17.78 0 180) (size 2 2) (drill 1) (layers *.Cu *.Mask) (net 30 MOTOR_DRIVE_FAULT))
  (pad 9 thru_hole circle (at 17.78 -10.16 180) (size 2 2) (drill 1) (layers *.Cu *.Mask) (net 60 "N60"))
  (pad 10 thru_hole circle (at 15.24 -10.16 180) (size 2 2) (drill 1) (layers *.Cu *.Mask) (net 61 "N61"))
  (pad 11 thru_hole circle (at 12.7 -10.16 180) (size 2 2) (drill 1) (layers *.Cu *.Mask) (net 8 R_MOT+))
  (pad 12 thru_hole circle (at 10.16 -10.16 180) (size 2 2) (drill 1) (layers *.Cu *.Mask) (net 9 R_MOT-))
  (pad 13 thru_hole circle (at 7.62 -10.16 180) (size 2 2) (drill 1) (layers *.Cu *.Mask) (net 7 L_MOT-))
  (pad 14 thru_hole circle (at 5.08 -10.16 180) (size 2 2) (drill 1) (layers *.Cu *.Mask) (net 6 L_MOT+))
  (pad 15 thru_hole circle (at 2.54 -10.16 180) (size 2 2) (drill 1) (layers *.Cu *.Mask) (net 1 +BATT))
  (pad 16 thru_hole circle (at 0 -10.16 180) (size 2 2) (drill 1) (layers *.Cu *.Mask) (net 2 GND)))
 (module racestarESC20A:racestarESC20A (layer F.Cu) (at 89 90)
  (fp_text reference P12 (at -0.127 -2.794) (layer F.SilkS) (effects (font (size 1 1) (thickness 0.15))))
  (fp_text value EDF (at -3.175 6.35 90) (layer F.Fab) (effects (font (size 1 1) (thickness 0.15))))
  (pad 1 thru_hole circle (at 0 0) (size 3.5 3.5) (drill 2) (layers *.Cu *.Mask) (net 1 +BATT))
  (pad 4 thru_hole circle (at 0 10.16) (size 3.5 3.5) (drill 2) (layers *.Cu *.Mask) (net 2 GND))
  (pad 2 thru_hole circle (at 0 3.81) (size 2 2) (drill 1) (layers *.Cu *.Mask) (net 50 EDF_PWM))
  (pad 3 thru_hole circle (at 0 6.35) (size 2 2) (drill 1) (layers *.Cu *.Mask) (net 2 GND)))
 (gr_line (start 200 96) (end 200 121) (angle 90) (layer Edge.Cuts) (width 0.1))
 (gr_line (start 160 56) (end 80 56) (angle 90) (layer Edge.Cuts) (width 0.1))
 (gr_line (start 168 64) (end 160 56) (angle 90) (layer Edge.Cuts) (width 0.1))
 (gr_line (start 200 96) (end 168 64) (angle 90) (layer Edge.Cuts) (width 0.1))
 (gr_line (start 40 96) (end 40 120) (angle 90) (layer Edge.Cuts) (width 0.1))
 (gr_line (start 72 64) (end 80 56) (angle 90) (layer Edge.Cuts) (width 0.1))
 (gr_line (start 40 96) (end 72 64) (angle 90) (layer Edge.Cuts) (width 0.1))
 (gr_line (start 60 120) (end 40 120) (angle 90) (layer Edge.Cuts) (width 0.1))
 (gr_line (start 60 156) (end 60 120) (angle 90) (layer Edge.Cuts) (width 0.1))
 (gr_line (start 60 156) (end 180 156) (angle 90) (layer Edge.Cuts) (width 0.1))
 (gr_line (start 180 121) (end 200 121) (angle 90) (layer Edge.Cuts) (width 0.1))
 (gr_line (start 180 156) (end 180 121) (angle 90) (layer Edge.Cuts) (width 0.1))
 (gr_circle (center 120.55 86.23) (end 138.33 84.96) (layer Edge.Cuts) (width 0.1))
 (segment (start 73.3 108) (end 73.3 110.765) (width 0.25) (layer B.Cu) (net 43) (status 400000))
 (segment (start 127.64 125.09) (end 127.64 122.87) (width 0.25) (layer B.Cu) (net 43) (status 800000))
 (segment (start 123.19 129.54) (end 127.64 125.09) (width 0.25) (layer B.Cu) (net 43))
 (segment (start 100.965 129.54) (end 123.19 129.54) (width 0.25) (layer B.Cu) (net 43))
 (segment (start 95.885 124.46) (end 100.965 129.54) (width 0.25) (layer B.Cu) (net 43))
 (segment (start 95.885 118.11) (end 95.885 124.46) (width 0.25) (layer B.Cu) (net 43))
 (segment (start 92.075 114.3) (end 95.885 118.11) (width 0.25) (layer B.Cu) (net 43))
 (segment (start 76.835 114.3) (end 92.075 114.3) (width 0.25) (layer B.Cu) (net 43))
 (segment (start 73.3 110.765) (end 76.835 114.3) (width 0.25) (layer B.Cu) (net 43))
 (segment (start 75.84 108) (end 75.84 110.765) (width 0.25) (layer B.Cu) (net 42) (status 400000))
 (segment (start 125.1 125.09) (end 125.1 122.87) (width 0.25) (layer B.Cu) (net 42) (status 800000))
 (segment (start 121.92 128.27) (end 125.1 125.09) (width 0.25) (layer B.Cu) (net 42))
 (segment (start 100.965 128.27) (end 121.92 128.27) (width 0.25) (layer B.Cu) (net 42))
 (segment (start 97.155 124.46) (end 100.965 128.27) (width 0.25) (layer B.Cu) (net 42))
 (segment (start 97.155 117.475) (end 97.155 124.46) (width 0.25) (layer B.Cu) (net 42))
 (segment (start 92.71 113.03) (end 97.155 117.475) (width 0.25) (layer B.Cu) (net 42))
 (segment (start 78.105 113.03) (end 92.71 113.03) (width 0.25) (layer B.Cu) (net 42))
 (segment (start 75.84 110.765) (end 78.105 113.03) (width 0.25) (layer B.Cu) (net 42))
 (segment (start 80.92 108) (end 80.92 110.215) (width 0.25) (layer B.Cu) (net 41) (status 400000))
 (segment (start 122.56 124.455) (end 122.56 122.87) (width 0.25) (layer B.Cu) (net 41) (status 800000))
 (segment (start 121.285 125.73) (end 122.56 124.455) (width 0.25) (layer B.Cu) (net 41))
 (segment (start 100.965 125.73) (end 121.285 125.73) (width 0.25) (layer B.Cu) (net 41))
 (segment (start 99.695 124.46) (end 100.965 125.73) (width 0.25) (layer B.Cu) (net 41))
 (segment (start 99.695 115.57) (end 99.695 124.46) (width 0.25) (layer B.Cu) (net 41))
 (segment (start 94.615 110.49) (end 99.695 115.57) (width 0.25) (layer B.Cu) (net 41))
 (segment (start 81.195 110.49) (end 94.615 110.49) (width 0.25) (layer B.Cu) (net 41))
 (segment (start 80.92 110.215) (end 81.195 110.49) (width 0.25) (layer B.Cu) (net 41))
 (segment (start 78.38 108) (end 78.38 110.765) (width 0.25) (layer B.Cu) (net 40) (status 400000))
 (segment (start 100.965 127) (end 120.015 127) (width 0.25) (layer B.Cu) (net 40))
 (segment (start 98.425 124.46) (end 100.965 127) (width 0.25) (layer B.Cu) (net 40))
 (segment (start 98.425 116.205) (end 98.425 124.46) (width 0.25) (layer B.Cu) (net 40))
 (segment (start 93.98 111.76) (end 98.425 116.205) (width 0.25) (layer B.Cu) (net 40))
 (segment (start 79.375 111.76) (end 93.98 111.76) (width 0.25) (layer B.Cu) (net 40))
 (segment (start 78.38 110.765) (end 79.375 111.76) (width 0.25) (layer B.Cu) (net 40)))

